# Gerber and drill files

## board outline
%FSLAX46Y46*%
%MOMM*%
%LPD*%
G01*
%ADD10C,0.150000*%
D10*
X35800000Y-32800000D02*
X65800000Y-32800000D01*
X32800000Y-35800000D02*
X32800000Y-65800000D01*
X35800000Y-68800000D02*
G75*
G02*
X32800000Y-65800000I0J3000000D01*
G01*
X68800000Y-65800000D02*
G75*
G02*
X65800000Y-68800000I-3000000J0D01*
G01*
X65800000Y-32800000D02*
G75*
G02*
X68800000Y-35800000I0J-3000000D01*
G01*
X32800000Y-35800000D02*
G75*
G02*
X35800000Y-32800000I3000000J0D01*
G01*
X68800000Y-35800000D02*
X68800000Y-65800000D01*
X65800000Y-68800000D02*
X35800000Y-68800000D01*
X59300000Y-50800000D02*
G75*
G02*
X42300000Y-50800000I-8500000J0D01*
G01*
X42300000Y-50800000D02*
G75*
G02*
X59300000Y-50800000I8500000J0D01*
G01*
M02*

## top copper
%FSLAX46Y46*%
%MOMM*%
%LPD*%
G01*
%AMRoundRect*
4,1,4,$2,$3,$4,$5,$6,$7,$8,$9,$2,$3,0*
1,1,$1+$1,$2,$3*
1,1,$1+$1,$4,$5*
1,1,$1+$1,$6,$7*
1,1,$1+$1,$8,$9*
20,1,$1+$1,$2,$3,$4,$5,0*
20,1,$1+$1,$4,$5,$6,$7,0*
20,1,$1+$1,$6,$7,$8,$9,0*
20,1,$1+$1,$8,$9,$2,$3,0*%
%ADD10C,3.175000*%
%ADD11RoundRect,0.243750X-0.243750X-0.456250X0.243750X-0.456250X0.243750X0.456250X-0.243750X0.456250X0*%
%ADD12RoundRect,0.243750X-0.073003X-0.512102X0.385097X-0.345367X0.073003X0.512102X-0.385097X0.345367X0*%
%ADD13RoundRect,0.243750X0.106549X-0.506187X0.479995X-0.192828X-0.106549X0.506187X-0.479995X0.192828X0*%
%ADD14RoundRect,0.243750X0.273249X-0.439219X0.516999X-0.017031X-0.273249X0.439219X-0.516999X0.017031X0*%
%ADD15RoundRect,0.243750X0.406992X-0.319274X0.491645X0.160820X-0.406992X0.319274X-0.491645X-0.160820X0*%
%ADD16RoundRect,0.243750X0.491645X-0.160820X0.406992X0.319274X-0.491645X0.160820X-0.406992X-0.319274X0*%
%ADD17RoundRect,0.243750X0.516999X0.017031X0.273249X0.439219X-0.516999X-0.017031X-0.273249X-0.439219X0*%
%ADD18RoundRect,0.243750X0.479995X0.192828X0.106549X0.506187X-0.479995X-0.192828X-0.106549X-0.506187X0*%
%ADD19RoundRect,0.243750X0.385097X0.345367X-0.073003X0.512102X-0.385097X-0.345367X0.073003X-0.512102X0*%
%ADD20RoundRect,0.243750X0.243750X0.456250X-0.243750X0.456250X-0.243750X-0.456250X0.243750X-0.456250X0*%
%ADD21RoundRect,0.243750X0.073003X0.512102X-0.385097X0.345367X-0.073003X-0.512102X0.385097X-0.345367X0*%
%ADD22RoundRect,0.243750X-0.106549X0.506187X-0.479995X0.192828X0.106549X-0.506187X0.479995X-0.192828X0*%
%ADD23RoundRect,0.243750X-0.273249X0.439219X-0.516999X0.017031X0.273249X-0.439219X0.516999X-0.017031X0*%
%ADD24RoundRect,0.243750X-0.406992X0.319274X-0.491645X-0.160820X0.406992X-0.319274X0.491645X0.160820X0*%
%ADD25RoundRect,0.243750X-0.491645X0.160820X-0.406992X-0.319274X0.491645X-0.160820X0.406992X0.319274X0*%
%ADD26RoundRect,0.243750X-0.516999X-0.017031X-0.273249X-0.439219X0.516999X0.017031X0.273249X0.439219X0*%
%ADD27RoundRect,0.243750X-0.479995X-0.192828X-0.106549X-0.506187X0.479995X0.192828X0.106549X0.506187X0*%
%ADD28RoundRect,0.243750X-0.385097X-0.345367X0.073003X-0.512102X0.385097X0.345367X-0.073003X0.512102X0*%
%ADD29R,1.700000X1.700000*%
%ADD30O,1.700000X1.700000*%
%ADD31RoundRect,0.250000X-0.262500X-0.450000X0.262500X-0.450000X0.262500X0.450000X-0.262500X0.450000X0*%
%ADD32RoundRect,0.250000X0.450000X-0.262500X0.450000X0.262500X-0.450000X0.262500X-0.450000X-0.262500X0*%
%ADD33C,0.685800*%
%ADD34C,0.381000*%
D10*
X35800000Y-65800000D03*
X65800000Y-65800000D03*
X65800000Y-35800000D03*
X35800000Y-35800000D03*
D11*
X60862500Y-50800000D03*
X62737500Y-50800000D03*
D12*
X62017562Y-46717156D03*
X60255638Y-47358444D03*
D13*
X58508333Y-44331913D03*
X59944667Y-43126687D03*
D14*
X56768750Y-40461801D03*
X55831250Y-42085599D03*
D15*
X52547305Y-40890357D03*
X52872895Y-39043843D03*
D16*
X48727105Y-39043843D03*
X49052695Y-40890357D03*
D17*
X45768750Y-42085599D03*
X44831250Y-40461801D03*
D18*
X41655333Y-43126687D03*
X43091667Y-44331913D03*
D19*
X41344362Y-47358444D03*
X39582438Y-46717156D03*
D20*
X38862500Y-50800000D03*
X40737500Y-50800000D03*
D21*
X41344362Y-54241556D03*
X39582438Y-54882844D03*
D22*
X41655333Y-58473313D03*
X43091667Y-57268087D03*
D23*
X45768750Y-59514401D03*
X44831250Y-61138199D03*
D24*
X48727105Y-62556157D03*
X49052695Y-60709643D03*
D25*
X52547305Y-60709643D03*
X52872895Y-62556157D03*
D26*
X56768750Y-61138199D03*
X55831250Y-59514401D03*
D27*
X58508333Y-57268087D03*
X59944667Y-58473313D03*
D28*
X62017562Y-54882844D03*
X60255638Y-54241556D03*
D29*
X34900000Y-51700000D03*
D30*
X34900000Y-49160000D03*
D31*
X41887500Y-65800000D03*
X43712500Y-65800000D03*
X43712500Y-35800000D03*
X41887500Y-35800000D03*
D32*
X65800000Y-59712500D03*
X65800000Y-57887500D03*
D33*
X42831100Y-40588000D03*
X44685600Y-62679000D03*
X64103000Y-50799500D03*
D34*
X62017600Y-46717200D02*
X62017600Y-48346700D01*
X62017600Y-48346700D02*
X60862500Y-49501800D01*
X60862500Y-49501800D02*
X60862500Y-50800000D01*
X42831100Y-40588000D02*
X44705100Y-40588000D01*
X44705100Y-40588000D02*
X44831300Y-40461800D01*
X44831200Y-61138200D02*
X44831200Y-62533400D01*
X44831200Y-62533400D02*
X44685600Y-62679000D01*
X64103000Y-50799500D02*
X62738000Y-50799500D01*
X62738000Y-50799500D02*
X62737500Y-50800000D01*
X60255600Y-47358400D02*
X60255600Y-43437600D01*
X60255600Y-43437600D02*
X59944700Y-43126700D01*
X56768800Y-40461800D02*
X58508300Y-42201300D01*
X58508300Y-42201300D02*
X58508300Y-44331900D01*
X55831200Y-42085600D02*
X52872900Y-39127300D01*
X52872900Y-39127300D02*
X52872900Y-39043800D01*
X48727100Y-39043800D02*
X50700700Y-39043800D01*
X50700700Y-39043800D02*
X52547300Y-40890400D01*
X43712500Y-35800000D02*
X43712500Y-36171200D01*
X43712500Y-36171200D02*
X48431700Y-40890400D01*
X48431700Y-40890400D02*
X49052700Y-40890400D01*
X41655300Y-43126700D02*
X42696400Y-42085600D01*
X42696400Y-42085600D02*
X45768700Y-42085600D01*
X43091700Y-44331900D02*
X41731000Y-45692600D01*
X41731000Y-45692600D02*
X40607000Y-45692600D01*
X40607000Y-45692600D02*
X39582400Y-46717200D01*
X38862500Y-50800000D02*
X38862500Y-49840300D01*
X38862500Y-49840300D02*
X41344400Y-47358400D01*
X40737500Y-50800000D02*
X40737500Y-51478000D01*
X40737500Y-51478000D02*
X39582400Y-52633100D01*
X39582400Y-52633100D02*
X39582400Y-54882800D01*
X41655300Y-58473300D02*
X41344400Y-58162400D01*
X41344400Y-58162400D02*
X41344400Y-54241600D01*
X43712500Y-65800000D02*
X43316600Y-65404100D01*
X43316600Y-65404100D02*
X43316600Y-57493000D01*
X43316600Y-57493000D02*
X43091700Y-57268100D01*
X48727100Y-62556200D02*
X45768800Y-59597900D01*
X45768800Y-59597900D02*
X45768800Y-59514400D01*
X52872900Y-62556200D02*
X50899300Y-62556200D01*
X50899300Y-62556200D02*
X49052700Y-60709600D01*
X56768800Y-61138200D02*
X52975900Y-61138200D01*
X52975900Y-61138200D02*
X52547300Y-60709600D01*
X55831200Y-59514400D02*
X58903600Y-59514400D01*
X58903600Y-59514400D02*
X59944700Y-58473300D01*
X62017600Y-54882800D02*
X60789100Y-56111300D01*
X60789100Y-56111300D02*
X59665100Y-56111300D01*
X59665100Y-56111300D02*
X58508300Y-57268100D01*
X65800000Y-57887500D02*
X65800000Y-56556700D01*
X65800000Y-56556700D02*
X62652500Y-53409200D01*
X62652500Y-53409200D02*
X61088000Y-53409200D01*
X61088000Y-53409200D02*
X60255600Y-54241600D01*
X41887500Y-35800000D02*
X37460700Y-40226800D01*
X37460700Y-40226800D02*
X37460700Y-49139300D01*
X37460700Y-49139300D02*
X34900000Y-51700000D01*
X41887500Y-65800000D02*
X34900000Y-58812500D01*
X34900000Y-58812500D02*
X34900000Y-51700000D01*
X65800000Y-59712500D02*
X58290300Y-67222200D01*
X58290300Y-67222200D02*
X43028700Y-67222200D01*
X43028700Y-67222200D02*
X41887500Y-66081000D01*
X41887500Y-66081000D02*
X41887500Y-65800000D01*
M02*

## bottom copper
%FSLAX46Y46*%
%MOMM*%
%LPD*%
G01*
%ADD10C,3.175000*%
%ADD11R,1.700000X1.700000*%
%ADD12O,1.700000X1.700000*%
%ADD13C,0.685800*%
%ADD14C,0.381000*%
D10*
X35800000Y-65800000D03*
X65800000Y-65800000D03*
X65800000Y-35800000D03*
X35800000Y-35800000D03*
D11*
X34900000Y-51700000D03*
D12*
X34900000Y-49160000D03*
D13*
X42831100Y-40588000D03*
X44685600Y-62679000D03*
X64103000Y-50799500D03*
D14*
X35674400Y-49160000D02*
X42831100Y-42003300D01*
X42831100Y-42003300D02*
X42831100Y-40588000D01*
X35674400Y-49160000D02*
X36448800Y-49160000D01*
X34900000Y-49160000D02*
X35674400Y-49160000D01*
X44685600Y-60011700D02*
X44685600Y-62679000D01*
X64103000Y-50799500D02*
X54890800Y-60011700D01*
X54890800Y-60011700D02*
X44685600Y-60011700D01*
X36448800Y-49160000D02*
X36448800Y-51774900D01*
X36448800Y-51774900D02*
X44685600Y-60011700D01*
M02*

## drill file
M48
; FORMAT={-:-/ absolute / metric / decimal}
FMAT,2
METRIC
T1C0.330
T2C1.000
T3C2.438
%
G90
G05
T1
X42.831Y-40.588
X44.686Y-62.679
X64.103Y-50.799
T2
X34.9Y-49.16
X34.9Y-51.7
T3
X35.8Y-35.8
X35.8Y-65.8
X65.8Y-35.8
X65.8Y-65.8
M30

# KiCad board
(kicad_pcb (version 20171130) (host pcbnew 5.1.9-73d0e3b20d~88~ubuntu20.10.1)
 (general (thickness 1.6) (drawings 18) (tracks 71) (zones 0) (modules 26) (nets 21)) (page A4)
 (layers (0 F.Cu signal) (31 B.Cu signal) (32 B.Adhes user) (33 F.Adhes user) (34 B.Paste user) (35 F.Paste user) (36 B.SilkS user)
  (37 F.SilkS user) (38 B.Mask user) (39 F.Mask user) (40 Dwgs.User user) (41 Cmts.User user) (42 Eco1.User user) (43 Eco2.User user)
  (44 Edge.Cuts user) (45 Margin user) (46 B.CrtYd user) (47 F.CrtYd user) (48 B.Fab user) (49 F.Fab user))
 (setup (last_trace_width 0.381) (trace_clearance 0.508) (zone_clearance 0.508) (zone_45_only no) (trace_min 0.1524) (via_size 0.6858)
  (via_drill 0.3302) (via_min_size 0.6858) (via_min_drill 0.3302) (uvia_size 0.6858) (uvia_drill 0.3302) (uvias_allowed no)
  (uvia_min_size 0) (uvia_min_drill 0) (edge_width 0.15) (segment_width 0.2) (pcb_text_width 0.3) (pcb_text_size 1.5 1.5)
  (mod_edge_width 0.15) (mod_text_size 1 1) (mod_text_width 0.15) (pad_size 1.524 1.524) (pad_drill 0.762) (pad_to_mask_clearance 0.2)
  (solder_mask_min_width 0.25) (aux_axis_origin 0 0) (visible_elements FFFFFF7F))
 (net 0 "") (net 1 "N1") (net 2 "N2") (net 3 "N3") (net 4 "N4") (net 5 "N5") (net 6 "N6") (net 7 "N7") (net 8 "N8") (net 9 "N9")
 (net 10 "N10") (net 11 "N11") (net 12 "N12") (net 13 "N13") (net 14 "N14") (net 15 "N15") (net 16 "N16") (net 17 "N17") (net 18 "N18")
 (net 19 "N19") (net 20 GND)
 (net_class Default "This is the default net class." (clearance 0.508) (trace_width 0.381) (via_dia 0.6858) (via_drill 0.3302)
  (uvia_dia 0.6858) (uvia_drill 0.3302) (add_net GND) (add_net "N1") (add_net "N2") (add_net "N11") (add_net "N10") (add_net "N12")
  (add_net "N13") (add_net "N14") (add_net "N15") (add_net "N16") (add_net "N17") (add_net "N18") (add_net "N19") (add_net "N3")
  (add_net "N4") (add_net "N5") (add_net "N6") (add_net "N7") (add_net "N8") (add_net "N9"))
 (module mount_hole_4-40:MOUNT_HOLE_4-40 (layer F.Cu) (at 35.8 65.8)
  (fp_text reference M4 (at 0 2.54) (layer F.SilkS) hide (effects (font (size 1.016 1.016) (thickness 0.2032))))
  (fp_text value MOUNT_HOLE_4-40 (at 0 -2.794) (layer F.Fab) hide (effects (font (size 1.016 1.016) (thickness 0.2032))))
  (pad 1 thru_hole circle (at 0 0) (size 3.175 3.175) (drill 2.4384) (layers *.Cu *.Mask)))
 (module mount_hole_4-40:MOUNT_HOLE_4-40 (layer F.Cu) (at 65.8 65.8)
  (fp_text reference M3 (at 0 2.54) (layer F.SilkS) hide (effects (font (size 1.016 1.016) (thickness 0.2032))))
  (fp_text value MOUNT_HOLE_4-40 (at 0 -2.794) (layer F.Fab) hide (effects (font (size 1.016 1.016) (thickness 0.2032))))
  (pad 1 thru_hole circle (at 0 0) (size 3.175 3.175) (drill 2.4384) (layers *.Cu *.Mask)))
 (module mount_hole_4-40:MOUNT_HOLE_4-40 (layer F.Cu) (at 65.8 35.8)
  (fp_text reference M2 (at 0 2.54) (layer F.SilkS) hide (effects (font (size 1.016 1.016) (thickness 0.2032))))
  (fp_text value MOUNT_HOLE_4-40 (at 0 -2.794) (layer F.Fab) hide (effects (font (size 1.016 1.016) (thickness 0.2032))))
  (pad 1 thru_hole circle (at 0 0) (size 3.175 3.175) (drill 2.4384) (layers *.Cu *.Mask)))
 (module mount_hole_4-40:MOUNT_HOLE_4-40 (layer F.Cu) (at 35.8 35.8)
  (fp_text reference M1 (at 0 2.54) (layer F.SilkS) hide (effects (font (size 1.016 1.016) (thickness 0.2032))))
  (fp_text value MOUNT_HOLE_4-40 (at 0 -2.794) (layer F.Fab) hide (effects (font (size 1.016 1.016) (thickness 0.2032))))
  (pad 1 thru_hole circle (at 0 0) (size 3.175 3.175) (drill 2.4384) (layers *.Cu *.Mask)))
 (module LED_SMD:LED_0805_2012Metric (layer F.Cu) (at 61.8 50.8)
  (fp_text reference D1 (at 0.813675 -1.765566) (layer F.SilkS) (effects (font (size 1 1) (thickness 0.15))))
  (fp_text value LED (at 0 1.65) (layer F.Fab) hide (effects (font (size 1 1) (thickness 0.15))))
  (pad 1 smd roundrect (at -0.9375 0) (size 0.975 1.4) (layers F.Cu F.Paste F.Mask) (roundrect_rratio 0.25) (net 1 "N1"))
  (pad 2 smd roundrect (at 0.9375 0) (size 0.975 1.4) (layers F.Cu F.Paste F.Mask) (roundrect_rratio 0.25) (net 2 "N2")))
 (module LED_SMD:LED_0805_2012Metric (layer F.Cu) (at 61.1366 47.0378 20)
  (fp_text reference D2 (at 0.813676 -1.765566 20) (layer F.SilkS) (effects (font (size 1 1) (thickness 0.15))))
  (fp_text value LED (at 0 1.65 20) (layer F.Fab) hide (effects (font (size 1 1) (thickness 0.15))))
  (pad 2 smd roundrect (at 0.9375 0 20) (size 0.975 1.4) (layers F.Cu F.Paste F.Mask) (roundrect_rratio 0.25) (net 1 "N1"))
  (pad 1 smd roundrect (at -0.9375 0 20) (size 0.975 1.4) (layers F.Cu F.Paste F.Mask) (roundrect_rratio 0.25) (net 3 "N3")))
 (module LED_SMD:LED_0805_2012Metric (layer F.Cu) (at 59.2265 43.7293 40)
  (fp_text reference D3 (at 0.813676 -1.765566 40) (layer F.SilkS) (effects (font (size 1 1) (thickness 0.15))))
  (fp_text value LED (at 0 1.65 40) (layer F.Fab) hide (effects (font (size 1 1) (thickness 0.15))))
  (pad 1 smd roundrect (at -0.9375 0 40) (size 0.975 1.4) (layers F.Cu F.Paste F.Mask) (roundrect_rratio 0.25) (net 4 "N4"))
  (pad 2 smd roundrect (at 0.9375 0 40) (size 0.975 1.4) (layers F.Cu F.Paste F.Mask) (roundrect_rratio 0.25) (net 3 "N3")))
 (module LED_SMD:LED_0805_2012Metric (layer F.Cu) (at 56.3 41.2737 60)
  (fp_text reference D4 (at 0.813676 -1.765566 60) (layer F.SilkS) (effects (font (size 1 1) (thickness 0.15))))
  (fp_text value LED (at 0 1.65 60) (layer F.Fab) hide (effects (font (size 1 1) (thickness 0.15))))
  (pad 2 smd roundrect (at 0.9375 0 60) (size 0.975 1.4) (layers F.Cu F.Paste F.Mask) (roundrect_rratio 0.25) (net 4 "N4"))
  (pad 1 smd roundrect (at -0.9375 0 60) (size 0.975 1.4) (layers F.Cu F.Paste F.Mask) (roundrect_rratio 0.25) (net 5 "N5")))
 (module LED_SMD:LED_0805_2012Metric (layer F.Cu) (at 52.7101 39.9671 80)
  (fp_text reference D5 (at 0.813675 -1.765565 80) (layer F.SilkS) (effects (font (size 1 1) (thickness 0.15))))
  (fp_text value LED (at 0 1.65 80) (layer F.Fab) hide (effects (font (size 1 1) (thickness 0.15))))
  (pad 1 smd roundrect (at -0.9375 0 80) (size 0.975 1.4) (layers F.Cu F.Paste F.Mask) (roundrect_rratio 0.25) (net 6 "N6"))
  (pad 2 smd roundrect (at 0.9375 0 80) (size 0.975 1.4) (layers F.Cu F.Paste F.Mask) (roundrect_rratio 0.25) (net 5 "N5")))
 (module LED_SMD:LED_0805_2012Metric (layer F.Cu) (at 48.8899 39.9671 100)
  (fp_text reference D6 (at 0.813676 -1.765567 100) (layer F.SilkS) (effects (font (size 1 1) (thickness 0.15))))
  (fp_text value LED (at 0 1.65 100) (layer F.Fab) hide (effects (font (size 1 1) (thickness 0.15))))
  (pad 2 smd roundrect (at 0.9375 0 100) (size 0.975 1.4) (layers F.Cu F.Paste F.Mask) (roundrect_rratio 0.25) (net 6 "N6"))
  (pad 1 smd roundrect (at -0.9375 0 100) (size 0.975 1.4) (layers F.Cu F.Paste F.Mask) (roundrect_rratio 0.25) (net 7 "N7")))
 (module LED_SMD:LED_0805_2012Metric (layer F.Cu) (at 45.3 41.2737 120)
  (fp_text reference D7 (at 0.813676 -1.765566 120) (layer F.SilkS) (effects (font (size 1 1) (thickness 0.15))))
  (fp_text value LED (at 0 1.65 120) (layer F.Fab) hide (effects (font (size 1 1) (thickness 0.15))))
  (pad 1 smd roundrect (at -0.9375 0 120) (size 0.975 1.4) (layers F.Cu F.Paste F.Mask) (roundrect_rratio 0.25) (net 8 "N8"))
  (pad 2 smd roundrect (at 0.9375 0 120) (size 0.975 1.4) (layers F.Cu F.Paste F.Mask) (roundrect_rratio 0.25) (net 2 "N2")))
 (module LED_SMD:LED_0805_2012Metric (layer F.Cu) (at 42.3735 43.7293 140)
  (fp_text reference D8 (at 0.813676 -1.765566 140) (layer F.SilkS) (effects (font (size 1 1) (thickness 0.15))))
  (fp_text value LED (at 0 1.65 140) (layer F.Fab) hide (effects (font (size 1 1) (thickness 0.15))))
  (pad 2 smd roundrect (at 0.9375 0 140) (size 0.975 1.4) (layers F.Cu F.Paste F.Mask) (roundrect_rratio 0.25) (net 8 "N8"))
  (pad 1 smd roundrect (at -0.9375 0 140) (size 0.975 1.4) (layers F.Cu F.Paste F.Mask) (roundrect_rratio 0.25) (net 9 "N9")))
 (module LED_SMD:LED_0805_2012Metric (layer F.Cu) (at 40.4634 47.0378 160)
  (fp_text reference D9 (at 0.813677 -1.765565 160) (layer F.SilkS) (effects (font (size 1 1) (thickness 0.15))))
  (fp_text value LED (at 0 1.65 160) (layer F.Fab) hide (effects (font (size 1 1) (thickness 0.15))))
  (pad 1 smd roundrect (at -0.9375 0 160) (size 0.975 1.4) (layers F.Cu F.Paste F.Mask) (roundrect_rratio 0.25) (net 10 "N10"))
  (pad 2 smd roundrect (at 0.9375 0 160) (size 0.975 1.4) (layers F.Cu F.Paste F.Mask) (roundrect_rratio 0.25) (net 9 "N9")))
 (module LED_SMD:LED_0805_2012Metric (layer F.Cu) (at 39.8 50.8 180)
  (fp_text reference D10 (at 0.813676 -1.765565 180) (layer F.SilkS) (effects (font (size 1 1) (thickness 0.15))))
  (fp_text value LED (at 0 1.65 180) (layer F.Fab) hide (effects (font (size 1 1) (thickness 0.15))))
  (pad 2 smd roundrect (at 0.9375 0 180) (size 0.975 1.4) (layers F.Cu F.Paste F.Mask) (roundrect_rratio 0.25) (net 10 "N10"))
  (pad 1 smd roundrect (at -0.9375 0 180) (size 0.975 1.4) (layers F.Cu F.Paste F.Mask) (roundrect_rratio 0.25) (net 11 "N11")))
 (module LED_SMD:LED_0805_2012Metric (layer F.Cu) (at 40.4634 54.5622 200)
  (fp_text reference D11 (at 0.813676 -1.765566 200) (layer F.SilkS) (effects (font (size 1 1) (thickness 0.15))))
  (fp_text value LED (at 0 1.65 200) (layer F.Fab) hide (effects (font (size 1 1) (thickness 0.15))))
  (pad 1 smd roundrect (at -0.9375 0 200) (size 0.975 1.4) (layers F.Cu F.Paste F.Mask) (roundrect_rratio 0.25) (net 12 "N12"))
  (pad 2 smd roundrect (at 0.9375 0 200) (size 0.975 1.4) (layers F.Cu F.Paste F.Mask) (roundrect_rratio 0.25) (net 11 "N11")))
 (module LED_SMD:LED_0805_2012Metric (layer F.Cu) (at 42.3735 57.8707 220)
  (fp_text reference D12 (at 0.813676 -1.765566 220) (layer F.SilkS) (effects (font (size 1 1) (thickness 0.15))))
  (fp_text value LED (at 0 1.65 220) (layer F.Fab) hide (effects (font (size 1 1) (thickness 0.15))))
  (pad 2 smd roundrect (at 0.9375 0 220) (size 0.975 1.4) (layers F.Cu F.Paste F.Mask) (roundrect_rratio 0.25) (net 12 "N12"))
  (pad 1 smd roundrect (at -0.9375 0 220) (size 0.975 1.4) (layers F.Cu F.Paste F.Mask) (roundrect_rratio 0.25) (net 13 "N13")))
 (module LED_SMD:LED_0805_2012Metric (layer F.Cu) (at 45.3 60.3263 240)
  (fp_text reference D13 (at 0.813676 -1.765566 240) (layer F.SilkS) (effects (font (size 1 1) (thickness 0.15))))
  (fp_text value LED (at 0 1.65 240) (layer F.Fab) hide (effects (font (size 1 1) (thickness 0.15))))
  (pad 1 smd roundrect (at -0.9375 0 240) (size 0.975 1.4) (layers F.Cu F.Paste F.Mask) (roundrect_rratio 0.25) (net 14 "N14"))
  (pad 2 smd roundrect (at 0.9375 0 240) (size 0.975 1.4) (layers F.Cu F.Paste F.Mask) (roundrect_rratio 0.25) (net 2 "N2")))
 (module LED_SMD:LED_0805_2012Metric (layer F.Cu) (at 48.8899 61.6329 260)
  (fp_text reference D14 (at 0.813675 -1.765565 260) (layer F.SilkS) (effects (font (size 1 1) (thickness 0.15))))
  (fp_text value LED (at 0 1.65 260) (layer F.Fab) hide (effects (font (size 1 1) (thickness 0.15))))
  (pad 2 smd roundrect (at 0.9375 0 260) (size 0.975 1.4) (layers F.Cu F.Paste F.Mask) (roundrect_rratio 0.25) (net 14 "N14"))
  (pad 1 smd roundrect (at -0.9375 0 260) (size 0.975 1.4) (layers F.Cu F.Paste F.Mask) (roundrect_rratio 0.25) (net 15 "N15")))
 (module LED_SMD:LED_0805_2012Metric (layer F.Cu) (at 52.7101 61.6329 280)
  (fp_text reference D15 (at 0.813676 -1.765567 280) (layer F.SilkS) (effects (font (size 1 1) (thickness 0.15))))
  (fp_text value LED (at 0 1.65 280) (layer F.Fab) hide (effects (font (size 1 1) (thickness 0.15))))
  (pad 1 smd roundrect (at -0.9375 0 280) (size 0.975 1.4) (layers F.Cu F.Paste F.Mask) (roundrect_rratio 0.25) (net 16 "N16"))
  (pad 2 smd roundrect (at 0.9375 0 280) (size 0.975 1.4) (layers F.Cu F.Paste F.Mask) (roundrect_rratio 0.25) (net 15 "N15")))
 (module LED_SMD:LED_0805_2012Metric (layer F.Cu) (at 56.3 60.3263 300)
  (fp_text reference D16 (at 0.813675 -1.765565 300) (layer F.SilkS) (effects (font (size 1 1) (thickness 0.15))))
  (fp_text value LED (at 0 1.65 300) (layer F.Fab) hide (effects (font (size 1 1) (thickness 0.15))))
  (pad 2 smd roundrect (at 0.9375 0 300) (size 0.975 1.4) (layers F.Cu F.Paste F.Mask) (roundrect_rratio 0.25) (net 16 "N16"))
  (pad 1 smd roundrect (at -0.9375 0 300) (size 0.975 1.4) (layers F.Cu F.Paste F.Mask) (roundrect_rratio 0.25) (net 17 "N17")))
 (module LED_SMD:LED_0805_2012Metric (layer F.Cu) (at 59.2265 57.8707 320)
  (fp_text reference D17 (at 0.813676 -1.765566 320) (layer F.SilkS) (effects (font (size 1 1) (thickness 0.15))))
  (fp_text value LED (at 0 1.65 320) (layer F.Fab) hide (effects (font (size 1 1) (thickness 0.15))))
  (pad 1 smd roundrect (at -0.9375 0 320) (size 0.975 1.4) (layers F.Cu F.Paste F.Mask) (roundrect_rratio 0.25) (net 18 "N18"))
  (pad 2 smd roundrect (at 0.9375 0 320) (size 0.975 1.4) (layers F.Cu F.Paste F.Mask) (roundrect_rratio 0.25) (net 17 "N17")))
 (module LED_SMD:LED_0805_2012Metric (layer F.Cu) (at 61.1366 54.5622 340)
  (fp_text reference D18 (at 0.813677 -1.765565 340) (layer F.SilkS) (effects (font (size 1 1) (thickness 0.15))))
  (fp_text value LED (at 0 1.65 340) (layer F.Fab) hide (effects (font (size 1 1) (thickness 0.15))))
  (pad 2 smd roundrect (at 0.9375 0 340) (size 0.975 1.4) (layers F.Cu F.Paste F.Mask) (roundrect_rratio 0.25) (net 18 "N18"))
  (pad 1 smd roundrect (at -0.9375 0 340) (size 0.975 1.4) (layers F.Cu F.Paste F.Mask) (roundrect_rratio 0.25) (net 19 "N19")))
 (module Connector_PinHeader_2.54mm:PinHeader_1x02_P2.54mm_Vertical (layer B.Cu) (at 34.9 51.7)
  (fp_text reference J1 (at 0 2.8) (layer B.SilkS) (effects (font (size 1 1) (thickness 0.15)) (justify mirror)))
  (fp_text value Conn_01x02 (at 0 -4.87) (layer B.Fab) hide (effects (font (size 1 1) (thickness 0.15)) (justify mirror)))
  (pad 1 thru_hole rect (at 0 0) (size 1.7 1.7) (drill 1) (layers *.Cu *.Mask) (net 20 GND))
  (pad 2 thru_hole oval (at 0 -2.54) (size 1.7 1.7) (drill 1) (layers *.Cu *.Mask) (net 2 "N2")))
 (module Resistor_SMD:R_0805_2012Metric (layer F.Cu) (at 42.8 65.8)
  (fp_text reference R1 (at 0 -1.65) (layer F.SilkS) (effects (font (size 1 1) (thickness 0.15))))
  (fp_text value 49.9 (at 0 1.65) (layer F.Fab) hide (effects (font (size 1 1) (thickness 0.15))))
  (pad 1 smd roundrect (at -0.9125 0) (size 1.025 1.4) (layers F.Cu F.Paste F.Mask) (roundrect_rratio 0.243902) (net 20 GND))
  (pad 2 smd roundrect (at 0.9125 0) (size 1.025 1.4) (layers F.Cu F.Paste F.Mask) (roundrect_rratio 0.243902) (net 13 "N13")))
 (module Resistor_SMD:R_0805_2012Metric (layer F.Cu) (at 42.8 35.8)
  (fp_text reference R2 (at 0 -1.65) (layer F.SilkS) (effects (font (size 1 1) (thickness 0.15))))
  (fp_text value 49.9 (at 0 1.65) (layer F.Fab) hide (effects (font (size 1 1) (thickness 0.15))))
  (pad 2 smd roundrect (at 0.9125 0) (size 1.025 1.4) (layers F.Cu F.Paste F.Mask) (roundrect_rratio 0.243902) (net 7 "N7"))
  (pad 1 smd roundrect (at -0.9125 0) (size 1.025 1.4) (layers F.Cu F.Paste F.Mask) (roundrect_rratio 0.243902) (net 20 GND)))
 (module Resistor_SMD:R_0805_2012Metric (layer F.Cu) (at 65.8 58.8 90)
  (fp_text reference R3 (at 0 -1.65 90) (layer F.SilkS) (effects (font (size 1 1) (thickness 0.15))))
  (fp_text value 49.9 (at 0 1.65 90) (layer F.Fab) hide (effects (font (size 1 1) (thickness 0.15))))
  (pad 1 smd roundrect (at -0.9125 0 90) (size 1.025 1.4) (layers F.Cu F.Paste F.Mask) (roundrect_rratio 0.243902) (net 20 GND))
  (pad 2 smd roundrect (at 0.9125 0 90) (size 1.025 1.4) (layers F.Cu F.Paste F.Mask) (roundrect_rratio 0.243902) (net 19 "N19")))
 (gr_line (start 35.8 32.8) (end 65.8 32.8) (layer Edge.Cuts) (width 0.15))
 (gr_line (start 32.8 35.8) (end 32.8 65.8) (layer Edge.Cuts) (width 0.15))
 (gr_arc (start 35.8 65.8) (end 32.8 65.8) (angle -90) (layer Edge.Cuts) (width 0.15))
 (gr_arc (start 65.8 65.8) (end 65.8 68.8) (angle -90) (layer Edge.Cuts) (width 0.15))
 (gr_arc (start 65.8 35.8) (end 68.8 35.8) (angle -90) (layer Edge.Cuts) (width 0.15))
 (gr_arc (start 35.8 35.8) (end 35.8 32.8) (angle -90) (layer Edge.Cuts) (width 0.15))
 (gr_line (start 68.8 35.8) (end 68.8 65.8) (layer Edge.Cuts) (width 0.15))
 (gr_line (start 65.8 68.8) (end 35.8 68.8) (layer Edge.Cuts) (width 0.15))
 (gr_circle (center 50.8 50.8) (end 59.3 50.8) (layer Edge.Cuts) (width 0.15))
 (segment (start 62.0176 46.7172) (end 62.0176 48.3467) (width 0.381) (layer F.Cu) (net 1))
 (segment (start 62.0176 48.3467) (end 60.8625 49.5018) (width 0.381) (layer F.Cu) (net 1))
 (segment (start 60.8625 49.5018) (end 60.8625 50.8) (width 0.381) (layer F.Cu) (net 1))
 (segment (start 42.8311 40.588) (end 44.7051 40.588) (width 0.381) (layer F.Cu) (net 2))
 (segment (start 44.7051 40.588) (end 44.8313 40.4618) (width 0.381) (layer F.Cu) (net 2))
 (segment (start 35.6744 49.16) (end 42.8311 42.0033) (width 0.381) (layer B.Cu) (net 2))
 (segment (start 42.8311 42.0033) (end 42.8311 40.588) (width 0.381) (layer B.Cu) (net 2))
 (segment (start 35.6744 49.16) (end 36.4488 49.16) (width 0.381) (layer B.Cu) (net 2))
 (segment (start 34.9 49.16) (end 35.6744 49.16) (width 0.381) (layer B.Cu) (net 2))
 (segment (start 44.6856 60.0117) (end 44.6856 62.679) (width 0.381) (layer B.Cu) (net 2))
 (segment (start 64.103 50.7995) (end 54.8908 60.0117) (width 0.381) (layer B.Cu) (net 2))
 (segment (start 54.8908 60.0117) (end 44.6856 60.0117) (width 0.381) (layer B.Cu) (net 2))
 (segment (start 36.4488 49.16) (end 36.4488 51.7749) (width 0.381) (layer B.Cu) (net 2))
 (segment (start 36.4488 51.7749) (end 44.6856 60.0117) (width 0.381) (layer B.Cu) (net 2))
 (segment (start 44.8312 61.1382) (end 44.8312 62.5334) (width 0.381) (layer F.Cu) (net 2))
 (segment (start 44.8312 62.5334) (end 44.6856 62.679) (width 0.381) (layer F.Cu) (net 2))
 (segment (start 64.103 50.7995) (end 62.738 50.7995) (width 0.381) (layer F.Cu) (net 2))
 (segment (start 62.738 50.7995) (end 62.7375 50.8) (width 0.381) (layer F.Cu) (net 2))
 (via (at 42.8311 40.588) (size 0.6858) (layers F.Cu B.Cu) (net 2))
 (via (at 44.6856 62.679) (size 0.6858) (layers F.Cu B.Cu) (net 2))
 (via (at 64.103 50.7995) (size 0.6858) (layers F.Cu B.Cu) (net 2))
 (segment (start 60.2556 47.3584) (end 60.2556 43.4376) (width 0.381) (layer F.Cu) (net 3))
 (segment (start 60.2556 43.4376) (end 59.9447 43.1267) (width 0.381) (layer F.Cu) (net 3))
 (segment (start 56.7688 40.4618) (end 58.5083 42.2013) (width 0.381) (layer F.Cu) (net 4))
 (segment (start 58.5083 42.2013) (end 58.5083 44.3319) (width 0.381) (layer F.Cu) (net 4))
 (segment (start 55.8312 42.0856) (end 52.8729 39.1273) (width 0.381) (layer F.Cu) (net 5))
 (segment (start 52.8729 39.1273) (end 52.8729 39.0438) (width 0.381) (layer F.Cu) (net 5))
 (segment (start 48.7271 39.0438) (end 50.7007 39.0438) (width 0.381) (layer F.Cu) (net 6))
 (segment (start 50.7007 39.0438) (end 52.5473 40.8904) (width 0.381) (layer F.Cu) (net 6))
 (segment (start 43.7125 35.8) (end 43.7125 36.1712) (width 0.381) (layer F.Cu) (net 7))
 (segment (start 43.7125 36.1712) (end 48.4317 40.8904) (width 0.381) (layer F.Cu) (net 7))
 (segment (start 48.4317 40.8904) (end 49.0527 40.8904) (width 0.381) (layer F.Cu) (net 7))
 (segment (start 41.6553 43.1267) (end 42.6964 42.0856) (width 0.381) (layer F.Cu) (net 8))
 (segment (start 42.6964 42.0856) (end 45.7687 42.0856) (width 0.381) (layer F.Cu) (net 8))
 (segment (start 43.0917 44.3319) (end 41.731 45.6926) (width 0.381) (layer F.Cu) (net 9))
 (segment (start 41.731 45.6926) (end 40.607 45.6926) (width 0.381) (layer F.Cu) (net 9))
 (segment (start 40.607 45.6926) (end 39.5824 46.7172) (width 0.381) (layer F.Cu) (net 9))
 (segment (start 38.8625 50.8) (end 38.8625 49.8403) (width 0.381) (layer F.Cu) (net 10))
 (segment (start 38.8625 49.8403) (end 41.3444 47.3584) (width 0.381) (layer F.Cu) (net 10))
 (segment (start 40.7375 50.8) (end 40.7375 51.478) (width 0.381) (layer F.Cu) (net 11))
 (segment (start 40.7375 51.478) (end 39.5824 52.6331) (width 0.381) (layer F.Cu) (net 11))
 (segment (start 39.5824 52.6331) (end 39.5824 54.8828) (width 0.381) (layer F.Cu) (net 11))
 (segment (start 41.6553 58.4733) (end 41.3444 58.1624) (width 0.381) (layer F.Cu) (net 12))
 (segment (start 41.3444 58.1624) (end 41.3444 54.2416) (width 0.381) (layer F.Cu) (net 12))
 (segment (start 43.7125 65.8) (end 43.3166 65.4041) (width 0.381) (layer F.Cu) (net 13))
 (segment (start 43.3166 65.4041) (end 43.3166 57.493) (width 0.381) (layer F.Cu) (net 13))
 (segment (start 43.3166 57.493) (end 43.0917 57.2681) (width 0.381) (layer F.Cu) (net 13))
 (segment (start 48.7271 62.5562) (end 45.7688 59.5979) (width 0.381) (layer F.Cu) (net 14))
 (segment (start 45.7688 59.5979) (end 45.7688 59.5144) (width 0.381) (layer F.Cu) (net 14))
 (segment (start 52.8729 62.5562) (end 50.8993 62.5562) (width 0.381) (layer F.Cu) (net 15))
 (segment (start 50.8993 62.5562) (end 49.0527 60.7096) (width 0.381) (layer F.Cu) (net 15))
 (segment (start 56.7688 61.1382) (end 52.9759 61.1382) (width 0.381) (layer F.Cu) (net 16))
 (segment (start 52.9759 61.1382) (end 52.5473 60.7096) (width 0.381) (layer F.Cu) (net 16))
 (segment (start 55.8312 59.5144) (end 58.9036 59.5144) (width 0.381) (layer F.Cu) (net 17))
 (segment (start 58.9036 59.5144) (end 59.9447 58.4733) (width 0.381) (layer F.Cu) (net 17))
 (segment (start 62.0176 54.8828) (end 60.7891 56.1113) (width 0.381) (layer F.Cu) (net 18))
 (segment (start 60.7891 56.1113) (end 59.6651 56.1113) (width 0.381) (layer F.Cu) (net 18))
 (segment (start 59.6651 56.1113) (end 58.5083 57.2681) (width 0.381) (layer F.Cu) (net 18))
 (segment (start 65.8 57.8875) (end 65.8 56.5567) (width 0.381) (layer F.Cu) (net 19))
 (segment (start 65.8 56.5567) (end 62.6525 53.4092) (width 0.381) (layer F.Cu) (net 19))
 (segment (start 62.6525 53.4092) (end 61.088 53.4092) (width 0.381) (layer F.Cu) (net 19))
 (segment (start 61.088 53.4092) (end 60.2556 54.2416) (width 0.381) (layer F.Cu) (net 19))
 (segment (start 41.8875 35.8) (end 37.4607 40.2268) (width 0.381) (layer F.Cu) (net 20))
 (segment (start 37.4607 40.2268) (end 37.4607 49.1393) (width 0.381) (layer F.Cu) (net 20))
 (segment (start 37.4607 49.1393) (end 34.9 51.7) (width 0.381) (layer F.Cu) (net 20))
 (segment (start 41.8875 65.8) (end 34.9 58.8125) (width 0.381) (layer F.Cu) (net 20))
 (segment (start 34.9 58.8125) (end 34.9 51.7) (width 0.381) (layer F.Cu) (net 20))
 (segment (start 65.8 59.7125) (end 58.2903 67.2222) (width 0.381) (layer F.Cu) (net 20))
 (segment (start 58.2903 67.2222) (end 43.0287 67.2222) (width 0.381) (layer F.Cu) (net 20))
 (segment (start 43.0287 67.2222) (end 41.8875 66.081) (width 0.381) (layer F.Cu) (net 20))
 (segment (start 41.8875 66.081) (end 41.8875 65.8) (width 0.381) (layer F.Cu) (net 20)))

